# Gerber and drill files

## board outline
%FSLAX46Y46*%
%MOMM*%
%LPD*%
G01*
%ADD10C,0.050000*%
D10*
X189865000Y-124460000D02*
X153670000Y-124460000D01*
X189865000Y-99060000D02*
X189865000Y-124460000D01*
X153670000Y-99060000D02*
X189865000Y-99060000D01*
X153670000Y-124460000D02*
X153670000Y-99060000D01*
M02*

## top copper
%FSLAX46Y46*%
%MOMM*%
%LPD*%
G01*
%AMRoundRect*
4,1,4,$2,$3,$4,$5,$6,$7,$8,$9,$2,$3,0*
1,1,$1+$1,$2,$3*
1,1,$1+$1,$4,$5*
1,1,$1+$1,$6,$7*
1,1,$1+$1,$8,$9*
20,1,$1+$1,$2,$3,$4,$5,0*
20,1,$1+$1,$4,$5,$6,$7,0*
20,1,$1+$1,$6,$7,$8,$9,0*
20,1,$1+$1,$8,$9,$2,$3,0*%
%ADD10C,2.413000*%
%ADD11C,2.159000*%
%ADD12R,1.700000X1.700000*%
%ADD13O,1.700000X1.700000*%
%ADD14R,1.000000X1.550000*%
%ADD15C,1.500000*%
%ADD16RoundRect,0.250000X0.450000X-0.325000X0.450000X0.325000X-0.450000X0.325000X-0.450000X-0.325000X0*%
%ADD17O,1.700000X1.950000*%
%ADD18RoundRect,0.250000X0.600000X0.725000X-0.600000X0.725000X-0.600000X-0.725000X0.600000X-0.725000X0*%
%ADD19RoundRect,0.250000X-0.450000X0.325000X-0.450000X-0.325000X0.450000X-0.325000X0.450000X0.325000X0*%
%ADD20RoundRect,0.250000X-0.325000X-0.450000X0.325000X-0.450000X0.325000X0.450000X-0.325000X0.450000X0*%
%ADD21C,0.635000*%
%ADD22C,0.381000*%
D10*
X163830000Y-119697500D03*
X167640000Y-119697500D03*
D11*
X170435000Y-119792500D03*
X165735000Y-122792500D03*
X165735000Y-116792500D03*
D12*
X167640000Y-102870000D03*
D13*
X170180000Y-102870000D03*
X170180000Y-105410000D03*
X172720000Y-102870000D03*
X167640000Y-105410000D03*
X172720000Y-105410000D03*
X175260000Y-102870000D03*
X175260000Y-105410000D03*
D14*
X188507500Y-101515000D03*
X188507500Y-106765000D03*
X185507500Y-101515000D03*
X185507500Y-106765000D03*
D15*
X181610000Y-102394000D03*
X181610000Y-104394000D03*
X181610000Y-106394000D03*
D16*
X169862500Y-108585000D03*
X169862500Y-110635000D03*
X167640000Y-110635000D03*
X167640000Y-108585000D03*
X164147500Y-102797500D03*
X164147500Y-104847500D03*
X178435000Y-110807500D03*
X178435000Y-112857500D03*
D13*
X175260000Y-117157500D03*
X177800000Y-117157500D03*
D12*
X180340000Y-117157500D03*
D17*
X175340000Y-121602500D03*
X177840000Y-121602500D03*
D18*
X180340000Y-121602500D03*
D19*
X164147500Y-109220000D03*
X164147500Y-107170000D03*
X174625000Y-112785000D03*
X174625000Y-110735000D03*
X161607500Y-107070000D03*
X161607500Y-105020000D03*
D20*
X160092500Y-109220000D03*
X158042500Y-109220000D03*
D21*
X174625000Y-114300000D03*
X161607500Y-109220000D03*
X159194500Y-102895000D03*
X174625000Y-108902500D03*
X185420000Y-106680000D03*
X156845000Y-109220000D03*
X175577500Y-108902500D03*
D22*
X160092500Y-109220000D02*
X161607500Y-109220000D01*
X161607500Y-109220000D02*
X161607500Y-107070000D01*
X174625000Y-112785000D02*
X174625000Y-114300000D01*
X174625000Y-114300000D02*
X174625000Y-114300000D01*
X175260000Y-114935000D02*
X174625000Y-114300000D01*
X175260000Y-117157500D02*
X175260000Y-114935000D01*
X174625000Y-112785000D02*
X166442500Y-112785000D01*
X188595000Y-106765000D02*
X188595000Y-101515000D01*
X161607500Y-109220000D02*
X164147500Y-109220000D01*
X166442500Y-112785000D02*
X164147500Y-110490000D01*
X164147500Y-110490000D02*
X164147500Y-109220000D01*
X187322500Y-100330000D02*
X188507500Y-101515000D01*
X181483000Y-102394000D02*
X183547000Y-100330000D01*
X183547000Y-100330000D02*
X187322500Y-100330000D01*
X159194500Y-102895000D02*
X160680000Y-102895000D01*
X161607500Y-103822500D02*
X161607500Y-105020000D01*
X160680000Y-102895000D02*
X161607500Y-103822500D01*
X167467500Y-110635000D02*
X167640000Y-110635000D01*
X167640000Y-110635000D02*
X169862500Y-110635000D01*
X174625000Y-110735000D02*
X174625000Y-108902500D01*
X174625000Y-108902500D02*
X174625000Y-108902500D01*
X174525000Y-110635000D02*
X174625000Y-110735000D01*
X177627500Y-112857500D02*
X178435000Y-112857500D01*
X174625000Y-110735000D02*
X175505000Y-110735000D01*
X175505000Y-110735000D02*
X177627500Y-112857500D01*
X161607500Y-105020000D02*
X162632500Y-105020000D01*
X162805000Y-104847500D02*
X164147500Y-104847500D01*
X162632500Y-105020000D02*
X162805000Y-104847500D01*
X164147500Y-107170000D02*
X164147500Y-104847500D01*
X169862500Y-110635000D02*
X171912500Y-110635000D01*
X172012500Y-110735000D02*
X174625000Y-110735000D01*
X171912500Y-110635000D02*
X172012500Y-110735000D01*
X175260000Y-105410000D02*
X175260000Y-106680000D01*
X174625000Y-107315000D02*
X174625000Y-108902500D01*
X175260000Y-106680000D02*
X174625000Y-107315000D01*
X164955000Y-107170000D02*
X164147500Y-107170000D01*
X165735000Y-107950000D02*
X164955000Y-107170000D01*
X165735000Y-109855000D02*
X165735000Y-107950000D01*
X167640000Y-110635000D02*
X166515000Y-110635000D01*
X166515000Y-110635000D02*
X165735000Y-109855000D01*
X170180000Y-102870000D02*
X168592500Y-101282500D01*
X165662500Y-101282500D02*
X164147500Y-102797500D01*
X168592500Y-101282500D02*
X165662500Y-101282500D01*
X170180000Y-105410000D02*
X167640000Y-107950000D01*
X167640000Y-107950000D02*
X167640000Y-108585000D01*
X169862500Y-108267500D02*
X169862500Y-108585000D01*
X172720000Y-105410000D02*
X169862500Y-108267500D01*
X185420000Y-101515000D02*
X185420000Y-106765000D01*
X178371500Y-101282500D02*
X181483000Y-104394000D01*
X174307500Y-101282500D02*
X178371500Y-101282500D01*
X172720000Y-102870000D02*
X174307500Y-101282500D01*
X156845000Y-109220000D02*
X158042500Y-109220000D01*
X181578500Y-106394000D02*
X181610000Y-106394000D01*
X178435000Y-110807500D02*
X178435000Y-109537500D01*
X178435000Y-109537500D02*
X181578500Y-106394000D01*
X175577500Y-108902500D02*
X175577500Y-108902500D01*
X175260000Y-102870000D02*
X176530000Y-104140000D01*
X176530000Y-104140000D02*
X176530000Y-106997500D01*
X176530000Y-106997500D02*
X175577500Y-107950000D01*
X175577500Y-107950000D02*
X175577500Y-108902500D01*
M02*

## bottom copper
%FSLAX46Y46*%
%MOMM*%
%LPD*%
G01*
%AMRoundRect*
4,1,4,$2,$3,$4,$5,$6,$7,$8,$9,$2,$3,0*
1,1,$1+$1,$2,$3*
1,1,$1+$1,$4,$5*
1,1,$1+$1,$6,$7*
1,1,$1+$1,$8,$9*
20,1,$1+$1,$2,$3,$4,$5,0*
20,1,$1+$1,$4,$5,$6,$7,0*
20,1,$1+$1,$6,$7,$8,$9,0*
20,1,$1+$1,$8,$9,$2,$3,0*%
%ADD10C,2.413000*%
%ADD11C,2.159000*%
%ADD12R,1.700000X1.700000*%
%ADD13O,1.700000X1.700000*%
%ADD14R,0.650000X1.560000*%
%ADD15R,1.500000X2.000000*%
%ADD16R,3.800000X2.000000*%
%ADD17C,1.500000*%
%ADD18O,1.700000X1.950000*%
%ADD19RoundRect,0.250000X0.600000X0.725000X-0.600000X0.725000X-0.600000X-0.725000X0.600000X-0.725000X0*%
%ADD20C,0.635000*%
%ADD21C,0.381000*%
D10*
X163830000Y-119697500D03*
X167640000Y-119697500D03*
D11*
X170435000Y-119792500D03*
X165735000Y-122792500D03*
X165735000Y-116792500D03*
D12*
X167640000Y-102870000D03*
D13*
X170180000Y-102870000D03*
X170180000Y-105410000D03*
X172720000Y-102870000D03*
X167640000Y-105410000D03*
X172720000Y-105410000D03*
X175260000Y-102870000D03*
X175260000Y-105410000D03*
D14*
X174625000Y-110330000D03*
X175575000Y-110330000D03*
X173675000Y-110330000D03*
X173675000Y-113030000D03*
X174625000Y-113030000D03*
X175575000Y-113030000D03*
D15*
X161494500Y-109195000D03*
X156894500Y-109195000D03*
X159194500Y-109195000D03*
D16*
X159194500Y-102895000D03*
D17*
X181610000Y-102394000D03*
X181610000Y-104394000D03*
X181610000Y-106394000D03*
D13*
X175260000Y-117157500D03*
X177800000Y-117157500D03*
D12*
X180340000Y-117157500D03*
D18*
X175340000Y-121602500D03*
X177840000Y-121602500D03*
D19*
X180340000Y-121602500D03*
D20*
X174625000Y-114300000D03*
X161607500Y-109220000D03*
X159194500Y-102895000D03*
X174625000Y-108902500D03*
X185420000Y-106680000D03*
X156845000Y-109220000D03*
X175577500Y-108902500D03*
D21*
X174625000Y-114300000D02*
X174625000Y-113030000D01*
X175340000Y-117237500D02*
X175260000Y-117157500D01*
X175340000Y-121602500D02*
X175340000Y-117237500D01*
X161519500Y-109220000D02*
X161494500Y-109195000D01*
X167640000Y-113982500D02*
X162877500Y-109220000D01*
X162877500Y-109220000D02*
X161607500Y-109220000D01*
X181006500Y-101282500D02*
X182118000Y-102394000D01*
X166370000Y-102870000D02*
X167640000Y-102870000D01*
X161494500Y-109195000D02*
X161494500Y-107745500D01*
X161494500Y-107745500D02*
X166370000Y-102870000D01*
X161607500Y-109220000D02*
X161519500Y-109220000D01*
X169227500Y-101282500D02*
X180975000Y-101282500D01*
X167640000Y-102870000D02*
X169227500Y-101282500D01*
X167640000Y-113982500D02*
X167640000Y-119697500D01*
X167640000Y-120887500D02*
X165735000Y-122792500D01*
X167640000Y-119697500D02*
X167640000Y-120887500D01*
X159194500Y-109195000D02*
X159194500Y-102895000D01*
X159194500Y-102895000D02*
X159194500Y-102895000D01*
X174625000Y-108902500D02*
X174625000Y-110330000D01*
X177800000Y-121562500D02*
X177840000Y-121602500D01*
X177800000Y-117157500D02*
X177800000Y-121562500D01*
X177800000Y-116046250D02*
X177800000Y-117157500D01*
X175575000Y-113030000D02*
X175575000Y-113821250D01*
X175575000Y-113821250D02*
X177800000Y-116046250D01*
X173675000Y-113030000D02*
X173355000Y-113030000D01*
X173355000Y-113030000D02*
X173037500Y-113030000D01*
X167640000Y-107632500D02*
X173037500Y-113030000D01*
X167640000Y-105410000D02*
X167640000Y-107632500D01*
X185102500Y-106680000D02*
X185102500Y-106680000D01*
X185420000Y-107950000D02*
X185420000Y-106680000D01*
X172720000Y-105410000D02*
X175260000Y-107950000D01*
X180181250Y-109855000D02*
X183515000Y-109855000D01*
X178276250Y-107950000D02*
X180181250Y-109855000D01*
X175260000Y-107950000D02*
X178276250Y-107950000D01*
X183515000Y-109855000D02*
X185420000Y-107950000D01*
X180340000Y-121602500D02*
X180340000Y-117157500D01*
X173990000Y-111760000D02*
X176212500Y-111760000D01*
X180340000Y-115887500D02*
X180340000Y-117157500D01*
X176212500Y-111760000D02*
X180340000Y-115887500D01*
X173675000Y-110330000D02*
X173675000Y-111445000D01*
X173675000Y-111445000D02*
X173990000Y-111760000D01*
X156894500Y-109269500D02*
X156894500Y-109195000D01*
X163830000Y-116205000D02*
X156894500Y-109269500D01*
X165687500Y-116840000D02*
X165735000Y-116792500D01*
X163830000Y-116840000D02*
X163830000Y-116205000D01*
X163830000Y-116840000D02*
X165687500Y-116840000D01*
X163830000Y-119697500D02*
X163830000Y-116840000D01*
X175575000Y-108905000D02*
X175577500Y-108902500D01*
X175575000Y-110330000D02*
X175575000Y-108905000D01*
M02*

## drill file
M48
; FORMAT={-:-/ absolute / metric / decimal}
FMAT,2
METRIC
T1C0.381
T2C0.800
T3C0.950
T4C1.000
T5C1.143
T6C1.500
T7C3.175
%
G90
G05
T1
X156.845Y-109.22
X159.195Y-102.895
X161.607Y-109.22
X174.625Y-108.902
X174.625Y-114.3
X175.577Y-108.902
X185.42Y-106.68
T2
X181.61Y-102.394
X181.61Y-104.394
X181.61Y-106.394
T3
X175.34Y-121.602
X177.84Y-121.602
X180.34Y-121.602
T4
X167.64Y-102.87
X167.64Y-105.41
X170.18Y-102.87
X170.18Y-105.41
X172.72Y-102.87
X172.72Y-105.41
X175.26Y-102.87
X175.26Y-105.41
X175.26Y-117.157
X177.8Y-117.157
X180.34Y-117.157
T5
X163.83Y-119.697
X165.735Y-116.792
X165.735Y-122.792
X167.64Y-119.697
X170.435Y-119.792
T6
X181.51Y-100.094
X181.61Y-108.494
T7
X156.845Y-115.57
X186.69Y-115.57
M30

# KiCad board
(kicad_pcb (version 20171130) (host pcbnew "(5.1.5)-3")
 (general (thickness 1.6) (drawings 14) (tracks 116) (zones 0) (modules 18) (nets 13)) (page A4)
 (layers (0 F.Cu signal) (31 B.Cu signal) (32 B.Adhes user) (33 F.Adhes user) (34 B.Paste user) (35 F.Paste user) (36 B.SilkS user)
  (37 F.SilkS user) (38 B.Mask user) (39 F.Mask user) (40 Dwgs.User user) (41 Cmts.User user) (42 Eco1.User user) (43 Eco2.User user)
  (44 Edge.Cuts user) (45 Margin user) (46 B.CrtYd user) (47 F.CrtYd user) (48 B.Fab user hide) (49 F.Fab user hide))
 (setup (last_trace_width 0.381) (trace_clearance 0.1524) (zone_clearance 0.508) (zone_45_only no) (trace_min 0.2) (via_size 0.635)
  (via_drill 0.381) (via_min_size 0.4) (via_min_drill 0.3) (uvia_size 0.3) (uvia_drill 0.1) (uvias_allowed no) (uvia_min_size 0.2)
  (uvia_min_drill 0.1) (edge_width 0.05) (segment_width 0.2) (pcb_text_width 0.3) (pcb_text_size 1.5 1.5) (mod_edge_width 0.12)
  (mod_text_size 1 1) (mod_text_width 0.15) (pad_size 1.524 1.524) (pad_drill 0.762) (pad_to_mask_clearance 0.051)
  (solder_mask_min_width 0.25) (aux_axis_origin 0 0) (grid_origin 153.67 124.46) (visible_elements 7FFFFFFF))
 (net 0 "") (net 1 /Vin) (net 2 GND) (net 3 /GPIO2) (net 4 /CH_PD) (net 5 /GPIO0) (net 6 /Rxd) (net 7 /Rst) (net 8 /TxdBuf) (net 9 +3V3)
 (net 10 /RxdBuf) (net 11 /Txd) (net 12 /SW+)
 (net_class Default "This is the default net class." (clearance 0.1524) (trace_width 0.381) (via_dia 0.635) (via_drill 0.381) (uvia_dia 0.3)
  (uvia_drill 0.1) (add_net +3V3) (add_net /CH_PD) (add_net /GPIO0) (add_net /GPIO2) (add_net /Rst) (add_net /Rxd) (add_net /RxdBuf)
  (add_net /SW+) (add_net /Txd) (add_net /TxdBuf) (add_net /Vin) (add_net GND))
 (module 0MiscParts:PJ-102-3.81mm (layer F.Cu) (at 165.735 130.4925 90)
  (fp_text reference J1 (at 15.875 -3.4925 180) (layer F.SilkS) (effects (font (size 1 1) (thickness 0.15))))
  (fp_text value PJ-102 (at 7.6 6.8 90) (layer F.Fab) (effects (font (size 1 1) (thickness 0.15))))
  (pad 1 thru_hole circle (at 10.795 -1.905) (size 2.413 2.413) (drill 1.143) (layers *.Cu *.Mask) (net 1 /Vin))
  (pad 2 thru_hole circle (at 10.795 1.905) (size 2.413 2.413) (drill 1.143) (layers *.Cu *.Mask) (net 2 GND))
  (pad 3 thru_hole circle (at 10.7 4.7 90) (size 2.159 2.159) (drill 1.143) (layers *.Cu *.Mask))
  (pad 2 thru_hole circle (at 7.7 0 90) (size 2.159 2.159) (drill 1.143) (layers *.Cu *.Mask) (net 2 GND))
  (pad 1 thru_hole circle (at 13.7 0 90) (size 2.159 2.159) (drill 1.143) (layers *.Cu *.Mask) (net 1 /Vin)))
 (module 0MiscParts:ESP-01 (layer F.Cu) (at 167.64 105.41 90)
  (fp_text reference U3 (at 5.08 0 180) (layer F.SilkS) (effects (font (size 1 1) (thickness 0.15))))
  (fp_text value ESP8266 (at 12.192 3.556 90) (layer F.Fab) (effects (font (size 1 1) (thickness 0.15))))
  (pad 1 thru_hole rect (at 2.54 0 90) (size 1.7 1.7) (drill 1) (layers *.Cu *.Mask) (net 2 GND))
  (pad 3 thru_hole oval (at 2.54 2.54 90) (size 1.7 1.7) (drill 1) (layers *.Cu *.Mask) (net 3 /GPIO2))
  (pad 4 thru_hole oval (at 0 2.54 90) (size 1.7 1.7) (drill 1) (layers *.Cu *.Mask) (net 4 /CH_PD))
  (pad 5 thru_hole oval (at 2.54 5.08 90) (size 1.7 1.7) (drill 1) (layers *.Cu *.Mask) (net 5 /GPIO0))
  (pad 2 thru_hole oval (at 0 0 90) (size 1.7 1.7) (drill 1) (layers *.Cu *.Mask) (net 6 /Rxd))
  (pad 6 thru_hole oval (at 0 5.08 90) (size 1.7 1.7) (drill 1) (layers *.Cu *.Mask) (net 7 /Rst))
  (pad 7 thru_hole oval (at 2.54 7.62 90) (size 1.7 1.7) (drill 1) (layers *.Cu *.Mask) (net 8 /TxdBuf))
  (pad 8 thru_hole oval (at 0 7.62 90) (size 1.7 1.7) (drill 1) (layers *.Cu *.Mask) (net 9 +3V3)))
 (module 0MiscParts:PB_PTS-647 (layer F.Cu) (at 187.0075 104.14 90)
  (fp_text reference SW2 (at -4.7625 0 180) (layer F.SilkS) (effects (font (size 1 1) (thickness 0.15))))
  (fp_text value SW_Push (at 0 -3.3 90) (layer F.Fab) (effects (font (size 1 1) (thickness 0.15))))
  (pad 2 smd rect (at 2.625 1.5 90) (size 1.55 1) (layers F.Cu F.Paste F.Mask) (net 2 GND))
  (pad 2 smd rect (at -2.625 1.5 90) (size 1.55 1) (layers F.Cu F.Paste F.Mask) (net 2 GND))
  (pad 1 smd rect (at 2.625 -1.5 90) (size 1.55 1) (layers F.Cu F.Paste F.Mask) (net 7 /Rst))
  (pad 1 smd rect (at -2.625 -1.5 90) (size 1.55 1) (layers F.Cu F.Paste F.Mask) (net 7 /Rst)))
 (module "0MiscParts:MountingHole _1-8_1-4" (layer F.Cu) (at 186.69 115.57)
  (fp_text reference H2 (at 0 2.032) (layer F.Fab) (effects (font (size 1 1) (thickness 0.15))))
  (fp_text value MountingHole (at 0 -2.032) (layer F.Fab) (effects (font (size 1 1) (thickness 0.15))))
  (pad "" np_thru_hole circle (at 0 0) (size 3.175 3.175) (drill 3.175) (layers *.Cu *.Mask)))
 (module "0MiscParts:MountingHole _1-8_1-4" (layer F.Cu) (at 156.845 115.57)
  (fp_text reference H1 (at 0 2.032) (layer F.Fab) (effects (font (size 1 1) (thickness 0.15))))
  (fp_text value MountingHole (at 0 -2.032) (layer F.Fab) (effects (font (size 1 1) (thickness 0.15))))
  (pad "" np_thru_hole circle (at 0 0) (size 3.175 3.175) (drill 3.175) (layers *.Cu *.Mask)))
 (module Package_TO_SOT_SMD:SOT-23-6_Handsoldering (layer B.Cu) (at 174.625 111.68 90)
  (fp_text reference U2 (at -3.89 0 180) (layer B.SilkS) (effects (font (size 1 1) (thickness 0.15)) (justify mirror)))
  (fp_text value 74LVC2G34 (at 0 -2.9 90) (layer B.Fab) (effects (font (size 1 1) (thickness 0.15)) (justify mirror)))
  (pad 5 smd rect (at 1.35 0 90) (size 1.56 0.65) (layers B.Cu B.Paste B.Mask) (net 9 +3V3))
  (pad 6 smd rect (at 1.35 0.95 90) (size 1.56 0.65) (layers B.Cu B.Paste B.Mask) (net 8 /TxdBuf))
  (pad 4 smd rect (at 1.35 -0.95 90) (size 1.56 0.65) (layers B.Cu B.Paste B.Mask) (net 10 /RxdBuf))
  (pad 3 smd rect (at -1.35 -0.95 90) (size 1.56 0.65) (layers B.Cu B.Paste B.Mask) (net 6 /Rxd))
  (pad 2 smd rect (at -1.35 0 90) (size 1.56 0.65) (layers B.Cu B.Paste B.Mask) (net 2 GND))
  (pad 1 smd rect (at -1.35 0.95 90) (size 1.56 0.65) (layers B.Cu B.Paste B.Mask) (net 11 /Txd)))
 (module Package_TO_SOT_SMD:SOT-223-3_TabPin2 (layer B.Cu) (at 159.1945 106.045 90)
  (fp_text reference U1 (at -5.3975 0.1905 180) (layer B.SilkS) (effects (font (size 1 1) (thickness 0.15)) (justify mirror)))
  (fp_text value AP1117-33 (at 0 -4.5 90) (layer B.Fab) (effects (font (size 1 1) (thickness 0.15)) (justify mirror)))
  (pad 1 smd rect (at -3.15 2.3 90) (size 2 1.5) (layers B.Cu B.Paste B.Mask) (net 2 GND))
  (pad 3 smd rect (at -3.15 -2.3 90) (size 2 1.5) (layers B.Cu B.Paste B.Mask) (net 1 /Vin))
  (pad 2 smd rect (at -3.15 0 90) (size 2 1.5) (layers B.Cu B.Paste B.Mask) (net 9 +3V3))
  (pad 2 smd rect (at 3.15 0 90) (size 2 3.8) (layers B.Cu B.Paste B.Mask) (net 9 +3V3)))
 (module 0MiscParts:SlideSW (layer F.Cu) (at 181.61 104.394 90)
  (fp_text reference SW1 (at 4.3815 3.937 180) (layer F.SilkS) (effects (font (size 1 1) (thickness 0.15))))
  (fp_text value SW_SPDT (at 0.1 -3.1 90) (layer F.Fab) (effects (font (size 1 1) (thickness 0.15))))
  (pad "" np_thru_hole circle (at 4.3 -0.1 90) (size 1.5 1.5) (drill 1.5) (layers *.Cu *.Mask))
  (pad "" np_thru_hole circle (at -4.1 0 90) (size 1.5 1.5) (drill 1.5) (layers *.Cu *.Mask))
  (pad 3 thru_hole circle (at 2 0 90) (size 1.5 1.5) (drill 0.8) (layers *.Cu *.Mask) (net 2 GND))
  (pad 2 thru_hole circle (at 0 0 90) (size 1.5 1.5) (drill 0.8) (layers *.Cu *.Mask) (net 5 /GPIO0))
  (pad 1 thru_hole circle (at -2 0 90) (size 1.5 1.5) (drill 0.8) (layers *.Cu *.Mask) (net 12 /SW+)))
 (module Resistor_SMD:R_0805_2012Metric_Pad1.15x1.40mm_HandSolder (layer F.Cu) (at 169.8625 109.61 90)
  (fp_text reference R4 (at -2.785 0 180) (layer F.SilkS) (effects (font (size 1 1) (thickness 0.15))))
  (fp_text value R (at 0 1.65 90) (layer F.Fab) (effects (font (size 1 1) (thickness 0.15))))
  (pad 2 smd roundrect (at 1.025 0 90) (size 1.15 1.4) (layers F.Cu F.Paste F.Mask) (roundrect_rratio 0.217391) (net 7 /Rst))
  (pad 1 smd roundrect (at -1.025 0 90) (size 1.15 1.4) (layers F.Cu F.Paste F.Mask) (roundrect_rratio 0.217391) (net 9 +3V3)))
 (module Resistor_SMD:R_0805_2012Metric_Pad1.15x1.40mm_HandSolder (layer F.Cu) (at 167.64 109.61 90)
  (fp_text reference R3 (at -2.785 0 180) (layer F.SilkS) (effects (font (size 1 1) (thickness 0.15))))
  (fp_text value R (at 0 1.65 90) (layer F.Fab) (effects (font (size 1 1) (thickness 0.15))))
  (pad 1 smd roundrect (at -1.025 0 90) (size 1.15 1.4) (layers F.Cu F.Paste F.Mask) (roundrect_rratio 0.217391) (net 9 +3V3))
  (pad 2 smd roundrect (at 1.025 0 90) (size 1.15 1.4) (layers F.Cu F.Paste F.Mask) (roundrect_rratio 0.217391) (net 4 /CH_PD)))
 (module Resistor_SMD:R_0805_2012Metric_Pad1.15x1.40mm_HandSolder (layer F.Cu) (at 164.1475 103.8225 90)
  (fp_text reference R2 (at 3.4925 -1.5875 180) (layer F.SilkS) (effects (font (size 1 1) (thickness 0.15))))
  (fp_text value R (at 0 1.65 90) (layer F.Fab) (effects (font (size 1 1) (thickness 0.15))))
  (pad 2 smd roundrect (at 1.025 0 90) (size 1.15 1.4) (layers F.Cu F.Paste F.Mask) (roundrect_rratio 0.217391) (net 3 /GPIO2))
  (pad 1 smd roundrect (at -1.025 0 90) (size 1.15 1.4) (layers F.Cu F.Paste F.Mask) (roundrect_rratio 0.217391) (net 9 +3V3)))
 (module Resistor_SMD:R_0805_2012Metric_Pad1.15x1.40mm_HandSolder (layer F.Cu) (at 178.435 111.8325 90)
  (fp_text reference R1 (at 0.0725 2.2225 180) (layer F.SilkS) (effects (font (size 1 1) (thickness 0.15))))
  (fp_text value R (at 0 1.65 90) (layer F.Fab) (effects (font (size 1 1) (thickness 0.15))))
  (pad 2 smd roundrect (at 1.025 0 90) (size 1.15 1.4) (layers F.Cu F.Paste F.Mask) (roundrect_rratio 0.217391) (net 12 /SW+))
  (pad 1 smd roundrect (at -1.025 0 90) (size 1.15 1.4) (layers F.Cu F.Paste F.Mask) (roundrect_rratio 0.217391) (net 9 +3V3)))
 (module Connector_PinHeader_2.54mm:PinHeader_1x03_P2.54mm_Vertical (layer F.Cu) (at 180.34 117.1575 270)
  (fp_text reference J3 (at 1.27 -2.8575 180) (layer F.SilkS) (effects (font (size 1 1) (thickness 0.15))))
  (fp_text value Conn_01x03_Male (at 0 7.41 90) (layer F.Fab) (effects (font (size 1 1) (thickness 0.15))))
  (pad 3 thru_hole oval (at 0 5.08 270) (size 1.7 1.7) (drill 1) (layers *.Cu *.Mask) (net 2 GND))
  (pad 2 thru_hole oval (at 0 2.54 270) (size 1.7 1.7) (drill 1) (layers *.Cu *.Mask) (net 11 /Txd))
  (pad 1 thru_hole rect (at 0 0 270) (size 1.7 1.7) (drill 1) (layers *.Cu *.Mask) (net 10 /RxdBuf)))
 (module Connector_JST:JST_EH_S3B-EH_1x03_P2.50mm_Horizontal (layer F.Cu) (at 180.34 121.6025 180)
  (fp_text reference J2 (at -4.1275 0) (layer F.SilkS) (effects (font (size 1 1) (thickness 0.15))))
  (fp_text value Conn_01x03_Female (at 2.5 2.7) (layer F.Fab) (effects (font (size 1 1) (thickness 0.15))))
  (pad 3 thru_hole oval (at 5 0 180) (size 1.7 1.95) (drill 0.95) (layers *.Cu *.Mask) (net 2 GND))
  (pad 2 thru_hole oval (at 2.5 0 180) (size 1.7 1.95) (drill 0.95) (layers *.Cu *.Mask) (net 11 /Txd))
  (pad 1 thru_hole roundrect (at 0 0 180) (size 1.7 1.95) (drill 0.95) (layers *.Cu *.Mask) (roundrect_rratio 0.147059) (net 10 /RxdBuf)))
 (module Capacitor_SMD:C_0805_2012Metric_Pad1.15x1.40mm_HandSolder (layer F.Cu) (at 164.1475 108.195 270)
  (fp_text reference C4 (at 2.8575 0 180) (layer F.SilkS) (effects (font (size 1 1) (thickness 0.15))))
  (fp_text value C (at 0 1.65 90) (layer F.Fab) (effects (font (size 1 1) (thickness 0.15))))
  (pad 2 smd roundrect (at 1.025 0 270) (size 1.15 1.4) (layers F.Cu F.Paste F.Mask) (roundrect_rratio 0.217391) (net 2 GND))
  (pad 1 smd roundrect (at -1.025 0 270) (size 1.15 1.4) (layers F.Cu F.Paste F.Mask) (roundrect_rratio 0.217391) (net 9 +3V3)))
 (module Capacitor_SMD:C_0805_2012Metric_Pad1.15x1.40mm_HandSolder (layer F.Cu) (at 174.625 111.76 270)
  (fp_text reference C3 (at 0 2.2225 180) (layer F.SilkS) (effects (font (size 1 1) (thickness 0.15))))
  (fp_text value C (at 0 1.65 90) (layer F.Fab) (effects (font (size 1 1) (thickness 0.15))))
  (pad 2 smd roundrect (at 1.025 0 270) (size 1.15 1.4) (layers F.Cu F.Paste F.Mask) (roundrect_rratio 0.217391) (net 2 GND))
  (pad 1 smd roundrect (at -1.025 0 270) (size 1.15 1.4) (layers F.Cu F.Paste F.Mask) (roundrect_rratio 0.217391) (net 9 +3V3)))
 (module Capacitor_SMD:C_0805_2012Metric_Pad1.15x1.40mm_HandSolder (layer F.Cu) (at 161.6075 106.045 270)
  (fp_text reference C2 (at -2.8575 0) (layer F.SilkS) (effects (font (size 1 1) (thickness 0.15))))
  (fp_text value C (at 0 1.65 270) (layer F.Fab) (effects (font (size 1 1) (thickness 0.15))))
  (pad 2 smd roundrect (at 1.025 0 270) (size 1.15 1.4) (layers F.Cu F.Paste F.Mask) (roundrect_rratio 0.217391) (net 2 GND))
  (pad 1 smd roundrect (at -1.025 0 270) (size 1.15 1.4) (layers F.Cu F.Paste F.Mask) (roundrect_rratio 0.217391) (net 9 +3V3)))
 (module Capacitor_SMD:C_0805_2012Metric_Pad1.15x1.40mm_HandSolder (layer F.Cu) (at 159.0675 109.22)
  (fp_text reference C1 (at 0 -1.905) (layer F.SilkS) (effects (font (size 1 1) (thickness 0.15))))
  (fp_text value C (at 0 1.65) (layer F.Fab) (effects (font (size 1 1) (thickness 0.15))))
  (pad 2 smd roundrect (at 1.025 0) (size 1.15 1.4) (layers F.Cu F.Paste F.Mask) (roundrect_rratio 0.217391) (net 2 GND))
  (pad 1 smd roundrect (at -1.025 0) (size 1.15 1.4) (layers F.Cu F.Paste F.Mask) (roundrect_rratio 0.217391) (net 1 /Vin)))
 (gr_line (start 189.865 124.46) (end 153.67 124.46) (layer Edge.Cuts) (width 0.05))
 (gr_line (start 189.865 99.06) (end 189.865 124.46) (layer Edge.Cuts) (width 0.05))
 (gr_line (start 153.67 99.06) (end 189.865 99.06) (layer Edge.Cuts) (width 0.05))
 (gr_line (start 153.67 124.46) (end 153.67 99.06) (layer Edge.Cuts) (width 0.05))
 (segment (start 160.0925 109.22) (end 161.6075 109.22) (width 0.381) (layer F.Cu) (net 2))
 (segment (start 161.6075 109.22) (end 161.6075 107.07) (width 0.381) (layer F.Cu) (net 2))
 (segment (start 174.625 112.785) (end 174.625 114.3) (width 0.381) (layer F.Cu) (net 2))
 (segment (start 174.625 114.3) (end 174.625 114.3) (width 0.381) (layer F.Cu) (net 2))
 (via (at 174.625 114.3) (size 0.635) (drill 0.381) (layers F.Cu B.Cu) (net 2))
 (segment (start 174.625 114.3) (end 174.625 113.03) (width 0.381) (layer B.Cu) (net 2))
 (segment (start 175.34 117.2375) (end 175.26 117.1575) (width 0.381) (layer B.Cu) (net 2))
 (segment (start 175.34 121.6025) (end 175.34 117.2375) (width 0.381) (layer B.Cu) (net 2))
 (segment (start 175.26 114.935) (end 174.625 114.3) (width 0.381) (layer F.Cu) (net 2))
 (segment (start 175.26 117.1575) (end 175.26 114.935) (width 0.381) (layer F.Cu) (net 2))
 (segment (start 174.625 112.785) (end 166.4425 112.785) (width 0.381) (layer F.Cu) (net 2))
 (segment (start 161.5195 109.22) (end 161.4945 109.195) (width 0.381) (layer B.Cu) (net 2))
 (segment (start 167.64 113.9825) (end 162.8775 109.22) (width 0.381) (layer B.Cu) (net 2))
 (segment (start 162.8775 109.22) (end 161.6075 109.22) (width 0.381) (layer B.Cu) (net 2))
 (segment (start 188.595 106.765) (end 188.595 101.515) (width 0.381) (layer F.Cu) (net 2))
 (segment (start 161.6075 109.22) (end 164.1475 109.22) (width 0.381) (layer F.Cu) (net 2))
 (segment (start 166.4425 112.785) (end 164.1475 110.49) (width 0.381) (layer F.Cu) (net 2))
 (segment (start 164.1475 110.49) (end 164.1475 109.22) (width 0.381) (layer F.Cu) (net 2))
 (segment (start 181.0065 101.2825) (end 182.118 102.394) (width 0.381) (layer B.Cu) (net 2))
 (segment (start 166.37 102.87) (end 167.64 102.87) (width 0.381) (layer B.Cu) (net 2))
 (segment (start 161.4945 109.195) (end 161.4945 107.7455) (width 0.381) (layer B.Cu) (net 2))
 (segment (start 161.4945 107.7455) (end 166.37 102.87) (width 0.381) (layer B.Cu) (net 2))
 (segment (start 161.6075 109.22) (end 161.5195 109.22) (width 0.381) (layer B.Cu) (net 2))
 (via (at 161.6075 109.22) (size 0.635) (drill 0.381) (layers F.Cu B.Cu) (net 2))
 (segment (start 169.2275 101.2825) (end 180.975 101.2825) (width 0.381) (layer B.Cu) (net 2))
 (segment (start 167.64 102.87) (end 169.2275 101.2825) (width 0.381) (layer B.Cu) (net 2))
 (segment (start 187.3225 100.33) (end 188.5075 101.515) (width 0.381) (layer F.Cu) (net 2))
 (segment (start 181.483 102.394) (end 183.547 100.33) (width 0.381) (layer F.Cu) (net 2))
 (segment (start 183.547 100.33) (end 187.3225 100.33) (width 0.381) (layer F.Cu) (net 2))
 (segment (start 167.64 113.9825) (end 167.64 119.6975) (width 0.381) (layer B.Cu) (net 2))
 (segment (start 167.64 120.8875) (end 165.735 122.7925) (width 0.381) (layer B.Cu) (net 2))
 (segment (start 167.64 119.6975) (end 167.64 120.8875) (width 0.381) (layer B.Cu) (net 2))
 (segment (start 159.1945 109.195) (end 159.1945 102.895) (width 0.381) (layer B.Cu) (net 9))
 (segment (start 159.1945 102.895) (end 159.1945 102.895) (width 0.381) (layer B.Cu) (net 9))
 (via (at 159.1945 102.895) (size 0.635) (drill 0.381) (layers F.Cu B.Cu) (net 9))
 (segment (start 159.1945 102.895) (end 160.68 102.895) (width 0.381) (layer F.Cu) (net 9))
 (segment (start 161.6075 103.8225) (end 161.6075 105.02) (width 0.381) (layer F.Cu) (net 9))
 (segment (start 160.68 102.895) (end 161.6075 103.8225) (width 0.381) (layer F.Cu) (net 9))
 (segment (start 167.4675 110.635) (end 167.64 110.635) (width 0.381) (layer F.Cu) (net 9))
 (segment (start 167.64 110.635) (end 169.8625 110.635) (width 0.381) (layer F.Cu) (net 9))
 (segment (start 174.625 110.735) (end 174.625 108.9025) (width 0.381) (layer F.Cu) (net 9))
 (segment (start 174.625 108.9025) (end 174.625 108.9025) (width 0.381) (layer F.Cu) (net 9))
 (via (at 174.625 108.9025) (size 0.635) (drill 0.381) (layers F.Cu B.Cu) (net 9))
 (segment (start 174.525 110.635) (end 174.625 110.735) (width 0.381) (layer F.Cu) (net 9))
 (segment (start 177.6275 112.8575) (end 178.435 112.8575) (width 0.381) (layer F.Cu) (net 9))
 (segment (start 174.625 110.735) (end 175.505 110.735) (width 0.381) (layer F.Cu) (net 9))
 (segment (start 175.505 110.735) (end 177.6275 112.8575) (width 0.381) (layer F.Cu) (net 9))
 (segment (start 161.6075 105.02) (end 162.6325 105.02) (width 0.381) (layer F.Cu) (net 9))
 (segment (start 162.805 104.8475) (end 164.1475 104.8475) (width 0.381) (layer F.Cu) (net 9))
 (segment (start 162.6325 105.02) (end 162.805 104.8475) (width 0.381) (layer F.Cu) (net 9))
 (segment (start 164.1475 107.17) (end 164.1475 104.8475) (width 0.381) (layer F.Cu) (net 9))
 (segment (start 169.8625 110.635) (end 171.9125 110.635) (width 0.381) (layer F.Cu) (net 9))
 (segment (start 172.0125 110.735) (end 174.625 110.735) (width 0.381) (layer F.Cu) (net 9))
 (segment (start 171.9125 110.635) (end 172.0125 110.735) (width 0.381) (layer F.Cu) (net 9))
 (segment (start 175.26 105.41) (end 175.26 106.68) (width 0.381) (layer F.Cu) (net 9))
 (segment (start 174.625 107.315) (end 174.625 108.9025) (width 0.381) (layer F.Cu) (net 9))
 (segment (start 175.26 106.68) (end 174.625 107.315) (width 0.381) (layer F.Cu) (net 9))
 (segment (start 164.955 107.17) (end 164.1475 107.17) (width 0.381) (layer F.Cu) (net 9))
 (segment (start 165.735 107.95) (end 164.955 107.17) (width 0.381) (layer F.Cu) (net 9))
 (segment (start 165.735 109.855) (end 165.735 107.95) (width 0.381) (layer F.Cu) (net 9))
 (segment (start 167.64 110.635) (end 166.515 110.635) (width 0.381) (layer F.Cu) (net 9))
 (segment (start 166.515 110.635) (end 165.735 109.855) (width 0.381) (layer F.Cu) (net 9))
 (segment (start 174.625 108.9025) (end 174.625 110.33) (width 0.381) (layer B.Cu) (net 9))
 (segment (start 177.8 121.5625) (end 177.84 121.6025) (width 0.381) (layer B.Cu) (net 11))
 (segment (start 177.8 117.1575) (end 177.8 121.5625) (width 0.381) (layer B.Cu) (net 11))
 (segment (start 177.8 116.04625) (end 177.8 117.1575) (width 0.381) (layer B.Cu) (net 11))
 (segment (start 175.575 113.03) (end 175.575 113.82125) (width 0.381) (layer B.Cu) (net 11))
 (segment (start 175.575 113.82125) (end 177.8 116.04625) (width 0.381) (layer B.Cu) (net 11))
 (segment (start 173.675 113.03) (end 173.355 113.03) (width 0.381) (layer B.Cu) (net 6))
 (segment (start 173.355 113.03) (end 173.0375 113.03) (width 0.381) (layer B.Cu) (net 6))
 (segment (start 167.64 107.6325) (end 173.0375 113.03) (width 0.381) (layer B.Cu) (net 6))
 (segment (start 167.64 105.41) (end 167.64 107.6325) (width 0.381) (layer B.Cu) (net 6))
 (segment (start 170.18 102.87) (end 168.5925 101.2825) (width 0.381) (layer F.Cu) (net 3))
 (segment (start 165.6625 101.2825) (end 164.1475 102.7975) (width 0.381) (layer F.Cu) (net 3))
 (segment (start 168.5925 101.2825) (end 165.6625 101.2825) (width 0.381) (layer F.Cu) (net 3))
 (segment (start 170.18 105.41) (end 167.64 107.95) (width 0.381) (layer F.Cu) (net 4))
 (segment (start 167.64 107.95) (end 167.64 108.585) (width 0.381) (layer F.Cu) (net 4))
 (segment (start 169.8625 108.2675) (end 169.8625 108.585) (width 0.381) (layer F.Cu) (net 7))
 (segment (start 172.72 105.41) (end 169.8625 108.2675) (width 0.381) (layer F.Cu) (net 7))
 (segment (start 185.1025 106.68) (end 185.1025 106.68) (width 0.381) (layer B.Cu) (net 7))
 (via (at 185.42 106.68) (size 0.635) (drill 0.381) (layers F.Cu B.Cu) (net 7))
 (segment (start 185.42 101.515) (end 185.42 106.765) (width 0.381) (layer F.Cu) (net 7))
 (segment (start 185.42 107.95) (end 185.42 106.68) (width 0.381) (layer B.Cu) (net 7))
 (segment (start 172.72 105.41) (end 175.26 107.95) (width 0.381) (layer B.Cu) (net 7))
 (segment (start 180.18125 109.855) (end 183.515 109.855) (width 0.381) (layer B.Cu) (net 7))
 (segment (start 178.27625 107.95) (end 180.18125 109.855) (width 0.381) (layer B.Cu) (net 7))
 (segment (start 175.26 107.95) (end 178.27625 107.95) (width 0.381) (layer B.Cu) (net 7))
 (segment (start 183.515 109.855) (end 185.42 107.95) (width 0.381) (layer B.Cu) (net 7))
 (segment (start 178.3715 101.2825) (end 181.483 104.394) (width 0.381) (layer F.Cu) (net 5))
 (segment (start 174.3075 101.2825) (end 178.3715 101.2825) (width 0.381) (layer F.Cu) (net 5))
 (segment (start 172.72 102.87) (end 174.3075 101.2825) (width 0.381) (layer F.Cu) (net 5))
 (segment (start 180.34 121.6025) (end 180.34 117.1575) (width 0.381) (layer B.Cu) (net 10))
 (segment (start 173.99 111.76) (end 176.2125 111.76) (width 0.381) (layer B.Cu) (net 10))
 (segment (start 180.34 115.8875) (end 180.34 117.1575) (width 0.381) (layer B.Cu) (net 10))
 (segment (start 176.2125 111.76) (end 180.34 115.8875) (width 0.381) (layer B.Cu) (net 10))
 (segment (start 173.675 110.33) (end 173.675 111.445) (width 0.381) (layer B.Cu) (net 10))
 (segment (start 173.675 111.445) (end 173.99 111.76) (width 0.381) (layer B.Cu) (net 10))
 (via (at 156.845 109.22) (size 0.635) (drill 0.381) (layers F.Cu B.Cu) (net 1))
 (segment (start 156.845 109.22) (end 158.0425 109.22) (width 0.381) (layer F.Cu) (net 1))
 (segment (start 156.8945 109.2695) (end 156.8945 109.195) (width 0.381) (layer B.Cu) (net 1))
 (segment (start 163.83 116.205) (end 156.8945 109.2695) (width 0.381) (layer B.Cu) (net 1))
 (segment (start 165.6875 116.84) (end 165.735 116.7925) (width 0.381) (layer B.Cu) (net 1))
 (segment (start 163.83 116.84) (end 163.83 116.205) (width 0.381) (layer B.Cu) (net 1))
 (segment (start 163.83 116.84) (end 165.6875 116.84) (width 0.381) (layer B.Cu) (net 1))
 (segment (start 163.83 119.6975) (end 163.83 116.84) (width 0.381) (layer B.Cu) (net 1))
 (segment (start 181.5785 106.394) (end 181.61 106.394) (width 0.381) (layer F.Cu) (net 12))
 (segment (start 178.435 110.8075) (end 178.435 109.5375) (width 0.381) (layer F.Cu) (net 12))
 (segment (start 178.435 109.5375) (end 181.5785 106.394) (width 0.381) (layer F.Cu) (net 12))
 (segment (start 175.5775 108.9025) (end 175.5775 108.9025) (width 0.381) (layer F.Cu) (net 8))
 (via (at 175.5775 108.9025) (size 0.635) (drill 0.381) (layers F.Cu B.Cu) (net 8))
 (segment (start 175.575 108.905) (end 175.5775 108.9025) (width 0.381) (layer B.Cu) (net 8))
 (segment (start 175.575 110.33) (end 175.575 108.905) (width 0.381) (layer B.Cu) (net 8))
 (segment (start 175.26 102.87) (end 176.53 104.14) (width 0.381) (layer F.Cu) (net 8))
 (segment (start 176.53 104.14) (end 176.53 106.9975) (width 0.381) (layer F.Cu) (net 8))
 (segment (start 176.53 106.9975) (end 175.5775 107.95) (width 0.381) (layer F.Cu) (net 8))
 (segment (start 175.5775 107.95) (end 175.5775 108.9025) (width 0.381) (layer F.Cu) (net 8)))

